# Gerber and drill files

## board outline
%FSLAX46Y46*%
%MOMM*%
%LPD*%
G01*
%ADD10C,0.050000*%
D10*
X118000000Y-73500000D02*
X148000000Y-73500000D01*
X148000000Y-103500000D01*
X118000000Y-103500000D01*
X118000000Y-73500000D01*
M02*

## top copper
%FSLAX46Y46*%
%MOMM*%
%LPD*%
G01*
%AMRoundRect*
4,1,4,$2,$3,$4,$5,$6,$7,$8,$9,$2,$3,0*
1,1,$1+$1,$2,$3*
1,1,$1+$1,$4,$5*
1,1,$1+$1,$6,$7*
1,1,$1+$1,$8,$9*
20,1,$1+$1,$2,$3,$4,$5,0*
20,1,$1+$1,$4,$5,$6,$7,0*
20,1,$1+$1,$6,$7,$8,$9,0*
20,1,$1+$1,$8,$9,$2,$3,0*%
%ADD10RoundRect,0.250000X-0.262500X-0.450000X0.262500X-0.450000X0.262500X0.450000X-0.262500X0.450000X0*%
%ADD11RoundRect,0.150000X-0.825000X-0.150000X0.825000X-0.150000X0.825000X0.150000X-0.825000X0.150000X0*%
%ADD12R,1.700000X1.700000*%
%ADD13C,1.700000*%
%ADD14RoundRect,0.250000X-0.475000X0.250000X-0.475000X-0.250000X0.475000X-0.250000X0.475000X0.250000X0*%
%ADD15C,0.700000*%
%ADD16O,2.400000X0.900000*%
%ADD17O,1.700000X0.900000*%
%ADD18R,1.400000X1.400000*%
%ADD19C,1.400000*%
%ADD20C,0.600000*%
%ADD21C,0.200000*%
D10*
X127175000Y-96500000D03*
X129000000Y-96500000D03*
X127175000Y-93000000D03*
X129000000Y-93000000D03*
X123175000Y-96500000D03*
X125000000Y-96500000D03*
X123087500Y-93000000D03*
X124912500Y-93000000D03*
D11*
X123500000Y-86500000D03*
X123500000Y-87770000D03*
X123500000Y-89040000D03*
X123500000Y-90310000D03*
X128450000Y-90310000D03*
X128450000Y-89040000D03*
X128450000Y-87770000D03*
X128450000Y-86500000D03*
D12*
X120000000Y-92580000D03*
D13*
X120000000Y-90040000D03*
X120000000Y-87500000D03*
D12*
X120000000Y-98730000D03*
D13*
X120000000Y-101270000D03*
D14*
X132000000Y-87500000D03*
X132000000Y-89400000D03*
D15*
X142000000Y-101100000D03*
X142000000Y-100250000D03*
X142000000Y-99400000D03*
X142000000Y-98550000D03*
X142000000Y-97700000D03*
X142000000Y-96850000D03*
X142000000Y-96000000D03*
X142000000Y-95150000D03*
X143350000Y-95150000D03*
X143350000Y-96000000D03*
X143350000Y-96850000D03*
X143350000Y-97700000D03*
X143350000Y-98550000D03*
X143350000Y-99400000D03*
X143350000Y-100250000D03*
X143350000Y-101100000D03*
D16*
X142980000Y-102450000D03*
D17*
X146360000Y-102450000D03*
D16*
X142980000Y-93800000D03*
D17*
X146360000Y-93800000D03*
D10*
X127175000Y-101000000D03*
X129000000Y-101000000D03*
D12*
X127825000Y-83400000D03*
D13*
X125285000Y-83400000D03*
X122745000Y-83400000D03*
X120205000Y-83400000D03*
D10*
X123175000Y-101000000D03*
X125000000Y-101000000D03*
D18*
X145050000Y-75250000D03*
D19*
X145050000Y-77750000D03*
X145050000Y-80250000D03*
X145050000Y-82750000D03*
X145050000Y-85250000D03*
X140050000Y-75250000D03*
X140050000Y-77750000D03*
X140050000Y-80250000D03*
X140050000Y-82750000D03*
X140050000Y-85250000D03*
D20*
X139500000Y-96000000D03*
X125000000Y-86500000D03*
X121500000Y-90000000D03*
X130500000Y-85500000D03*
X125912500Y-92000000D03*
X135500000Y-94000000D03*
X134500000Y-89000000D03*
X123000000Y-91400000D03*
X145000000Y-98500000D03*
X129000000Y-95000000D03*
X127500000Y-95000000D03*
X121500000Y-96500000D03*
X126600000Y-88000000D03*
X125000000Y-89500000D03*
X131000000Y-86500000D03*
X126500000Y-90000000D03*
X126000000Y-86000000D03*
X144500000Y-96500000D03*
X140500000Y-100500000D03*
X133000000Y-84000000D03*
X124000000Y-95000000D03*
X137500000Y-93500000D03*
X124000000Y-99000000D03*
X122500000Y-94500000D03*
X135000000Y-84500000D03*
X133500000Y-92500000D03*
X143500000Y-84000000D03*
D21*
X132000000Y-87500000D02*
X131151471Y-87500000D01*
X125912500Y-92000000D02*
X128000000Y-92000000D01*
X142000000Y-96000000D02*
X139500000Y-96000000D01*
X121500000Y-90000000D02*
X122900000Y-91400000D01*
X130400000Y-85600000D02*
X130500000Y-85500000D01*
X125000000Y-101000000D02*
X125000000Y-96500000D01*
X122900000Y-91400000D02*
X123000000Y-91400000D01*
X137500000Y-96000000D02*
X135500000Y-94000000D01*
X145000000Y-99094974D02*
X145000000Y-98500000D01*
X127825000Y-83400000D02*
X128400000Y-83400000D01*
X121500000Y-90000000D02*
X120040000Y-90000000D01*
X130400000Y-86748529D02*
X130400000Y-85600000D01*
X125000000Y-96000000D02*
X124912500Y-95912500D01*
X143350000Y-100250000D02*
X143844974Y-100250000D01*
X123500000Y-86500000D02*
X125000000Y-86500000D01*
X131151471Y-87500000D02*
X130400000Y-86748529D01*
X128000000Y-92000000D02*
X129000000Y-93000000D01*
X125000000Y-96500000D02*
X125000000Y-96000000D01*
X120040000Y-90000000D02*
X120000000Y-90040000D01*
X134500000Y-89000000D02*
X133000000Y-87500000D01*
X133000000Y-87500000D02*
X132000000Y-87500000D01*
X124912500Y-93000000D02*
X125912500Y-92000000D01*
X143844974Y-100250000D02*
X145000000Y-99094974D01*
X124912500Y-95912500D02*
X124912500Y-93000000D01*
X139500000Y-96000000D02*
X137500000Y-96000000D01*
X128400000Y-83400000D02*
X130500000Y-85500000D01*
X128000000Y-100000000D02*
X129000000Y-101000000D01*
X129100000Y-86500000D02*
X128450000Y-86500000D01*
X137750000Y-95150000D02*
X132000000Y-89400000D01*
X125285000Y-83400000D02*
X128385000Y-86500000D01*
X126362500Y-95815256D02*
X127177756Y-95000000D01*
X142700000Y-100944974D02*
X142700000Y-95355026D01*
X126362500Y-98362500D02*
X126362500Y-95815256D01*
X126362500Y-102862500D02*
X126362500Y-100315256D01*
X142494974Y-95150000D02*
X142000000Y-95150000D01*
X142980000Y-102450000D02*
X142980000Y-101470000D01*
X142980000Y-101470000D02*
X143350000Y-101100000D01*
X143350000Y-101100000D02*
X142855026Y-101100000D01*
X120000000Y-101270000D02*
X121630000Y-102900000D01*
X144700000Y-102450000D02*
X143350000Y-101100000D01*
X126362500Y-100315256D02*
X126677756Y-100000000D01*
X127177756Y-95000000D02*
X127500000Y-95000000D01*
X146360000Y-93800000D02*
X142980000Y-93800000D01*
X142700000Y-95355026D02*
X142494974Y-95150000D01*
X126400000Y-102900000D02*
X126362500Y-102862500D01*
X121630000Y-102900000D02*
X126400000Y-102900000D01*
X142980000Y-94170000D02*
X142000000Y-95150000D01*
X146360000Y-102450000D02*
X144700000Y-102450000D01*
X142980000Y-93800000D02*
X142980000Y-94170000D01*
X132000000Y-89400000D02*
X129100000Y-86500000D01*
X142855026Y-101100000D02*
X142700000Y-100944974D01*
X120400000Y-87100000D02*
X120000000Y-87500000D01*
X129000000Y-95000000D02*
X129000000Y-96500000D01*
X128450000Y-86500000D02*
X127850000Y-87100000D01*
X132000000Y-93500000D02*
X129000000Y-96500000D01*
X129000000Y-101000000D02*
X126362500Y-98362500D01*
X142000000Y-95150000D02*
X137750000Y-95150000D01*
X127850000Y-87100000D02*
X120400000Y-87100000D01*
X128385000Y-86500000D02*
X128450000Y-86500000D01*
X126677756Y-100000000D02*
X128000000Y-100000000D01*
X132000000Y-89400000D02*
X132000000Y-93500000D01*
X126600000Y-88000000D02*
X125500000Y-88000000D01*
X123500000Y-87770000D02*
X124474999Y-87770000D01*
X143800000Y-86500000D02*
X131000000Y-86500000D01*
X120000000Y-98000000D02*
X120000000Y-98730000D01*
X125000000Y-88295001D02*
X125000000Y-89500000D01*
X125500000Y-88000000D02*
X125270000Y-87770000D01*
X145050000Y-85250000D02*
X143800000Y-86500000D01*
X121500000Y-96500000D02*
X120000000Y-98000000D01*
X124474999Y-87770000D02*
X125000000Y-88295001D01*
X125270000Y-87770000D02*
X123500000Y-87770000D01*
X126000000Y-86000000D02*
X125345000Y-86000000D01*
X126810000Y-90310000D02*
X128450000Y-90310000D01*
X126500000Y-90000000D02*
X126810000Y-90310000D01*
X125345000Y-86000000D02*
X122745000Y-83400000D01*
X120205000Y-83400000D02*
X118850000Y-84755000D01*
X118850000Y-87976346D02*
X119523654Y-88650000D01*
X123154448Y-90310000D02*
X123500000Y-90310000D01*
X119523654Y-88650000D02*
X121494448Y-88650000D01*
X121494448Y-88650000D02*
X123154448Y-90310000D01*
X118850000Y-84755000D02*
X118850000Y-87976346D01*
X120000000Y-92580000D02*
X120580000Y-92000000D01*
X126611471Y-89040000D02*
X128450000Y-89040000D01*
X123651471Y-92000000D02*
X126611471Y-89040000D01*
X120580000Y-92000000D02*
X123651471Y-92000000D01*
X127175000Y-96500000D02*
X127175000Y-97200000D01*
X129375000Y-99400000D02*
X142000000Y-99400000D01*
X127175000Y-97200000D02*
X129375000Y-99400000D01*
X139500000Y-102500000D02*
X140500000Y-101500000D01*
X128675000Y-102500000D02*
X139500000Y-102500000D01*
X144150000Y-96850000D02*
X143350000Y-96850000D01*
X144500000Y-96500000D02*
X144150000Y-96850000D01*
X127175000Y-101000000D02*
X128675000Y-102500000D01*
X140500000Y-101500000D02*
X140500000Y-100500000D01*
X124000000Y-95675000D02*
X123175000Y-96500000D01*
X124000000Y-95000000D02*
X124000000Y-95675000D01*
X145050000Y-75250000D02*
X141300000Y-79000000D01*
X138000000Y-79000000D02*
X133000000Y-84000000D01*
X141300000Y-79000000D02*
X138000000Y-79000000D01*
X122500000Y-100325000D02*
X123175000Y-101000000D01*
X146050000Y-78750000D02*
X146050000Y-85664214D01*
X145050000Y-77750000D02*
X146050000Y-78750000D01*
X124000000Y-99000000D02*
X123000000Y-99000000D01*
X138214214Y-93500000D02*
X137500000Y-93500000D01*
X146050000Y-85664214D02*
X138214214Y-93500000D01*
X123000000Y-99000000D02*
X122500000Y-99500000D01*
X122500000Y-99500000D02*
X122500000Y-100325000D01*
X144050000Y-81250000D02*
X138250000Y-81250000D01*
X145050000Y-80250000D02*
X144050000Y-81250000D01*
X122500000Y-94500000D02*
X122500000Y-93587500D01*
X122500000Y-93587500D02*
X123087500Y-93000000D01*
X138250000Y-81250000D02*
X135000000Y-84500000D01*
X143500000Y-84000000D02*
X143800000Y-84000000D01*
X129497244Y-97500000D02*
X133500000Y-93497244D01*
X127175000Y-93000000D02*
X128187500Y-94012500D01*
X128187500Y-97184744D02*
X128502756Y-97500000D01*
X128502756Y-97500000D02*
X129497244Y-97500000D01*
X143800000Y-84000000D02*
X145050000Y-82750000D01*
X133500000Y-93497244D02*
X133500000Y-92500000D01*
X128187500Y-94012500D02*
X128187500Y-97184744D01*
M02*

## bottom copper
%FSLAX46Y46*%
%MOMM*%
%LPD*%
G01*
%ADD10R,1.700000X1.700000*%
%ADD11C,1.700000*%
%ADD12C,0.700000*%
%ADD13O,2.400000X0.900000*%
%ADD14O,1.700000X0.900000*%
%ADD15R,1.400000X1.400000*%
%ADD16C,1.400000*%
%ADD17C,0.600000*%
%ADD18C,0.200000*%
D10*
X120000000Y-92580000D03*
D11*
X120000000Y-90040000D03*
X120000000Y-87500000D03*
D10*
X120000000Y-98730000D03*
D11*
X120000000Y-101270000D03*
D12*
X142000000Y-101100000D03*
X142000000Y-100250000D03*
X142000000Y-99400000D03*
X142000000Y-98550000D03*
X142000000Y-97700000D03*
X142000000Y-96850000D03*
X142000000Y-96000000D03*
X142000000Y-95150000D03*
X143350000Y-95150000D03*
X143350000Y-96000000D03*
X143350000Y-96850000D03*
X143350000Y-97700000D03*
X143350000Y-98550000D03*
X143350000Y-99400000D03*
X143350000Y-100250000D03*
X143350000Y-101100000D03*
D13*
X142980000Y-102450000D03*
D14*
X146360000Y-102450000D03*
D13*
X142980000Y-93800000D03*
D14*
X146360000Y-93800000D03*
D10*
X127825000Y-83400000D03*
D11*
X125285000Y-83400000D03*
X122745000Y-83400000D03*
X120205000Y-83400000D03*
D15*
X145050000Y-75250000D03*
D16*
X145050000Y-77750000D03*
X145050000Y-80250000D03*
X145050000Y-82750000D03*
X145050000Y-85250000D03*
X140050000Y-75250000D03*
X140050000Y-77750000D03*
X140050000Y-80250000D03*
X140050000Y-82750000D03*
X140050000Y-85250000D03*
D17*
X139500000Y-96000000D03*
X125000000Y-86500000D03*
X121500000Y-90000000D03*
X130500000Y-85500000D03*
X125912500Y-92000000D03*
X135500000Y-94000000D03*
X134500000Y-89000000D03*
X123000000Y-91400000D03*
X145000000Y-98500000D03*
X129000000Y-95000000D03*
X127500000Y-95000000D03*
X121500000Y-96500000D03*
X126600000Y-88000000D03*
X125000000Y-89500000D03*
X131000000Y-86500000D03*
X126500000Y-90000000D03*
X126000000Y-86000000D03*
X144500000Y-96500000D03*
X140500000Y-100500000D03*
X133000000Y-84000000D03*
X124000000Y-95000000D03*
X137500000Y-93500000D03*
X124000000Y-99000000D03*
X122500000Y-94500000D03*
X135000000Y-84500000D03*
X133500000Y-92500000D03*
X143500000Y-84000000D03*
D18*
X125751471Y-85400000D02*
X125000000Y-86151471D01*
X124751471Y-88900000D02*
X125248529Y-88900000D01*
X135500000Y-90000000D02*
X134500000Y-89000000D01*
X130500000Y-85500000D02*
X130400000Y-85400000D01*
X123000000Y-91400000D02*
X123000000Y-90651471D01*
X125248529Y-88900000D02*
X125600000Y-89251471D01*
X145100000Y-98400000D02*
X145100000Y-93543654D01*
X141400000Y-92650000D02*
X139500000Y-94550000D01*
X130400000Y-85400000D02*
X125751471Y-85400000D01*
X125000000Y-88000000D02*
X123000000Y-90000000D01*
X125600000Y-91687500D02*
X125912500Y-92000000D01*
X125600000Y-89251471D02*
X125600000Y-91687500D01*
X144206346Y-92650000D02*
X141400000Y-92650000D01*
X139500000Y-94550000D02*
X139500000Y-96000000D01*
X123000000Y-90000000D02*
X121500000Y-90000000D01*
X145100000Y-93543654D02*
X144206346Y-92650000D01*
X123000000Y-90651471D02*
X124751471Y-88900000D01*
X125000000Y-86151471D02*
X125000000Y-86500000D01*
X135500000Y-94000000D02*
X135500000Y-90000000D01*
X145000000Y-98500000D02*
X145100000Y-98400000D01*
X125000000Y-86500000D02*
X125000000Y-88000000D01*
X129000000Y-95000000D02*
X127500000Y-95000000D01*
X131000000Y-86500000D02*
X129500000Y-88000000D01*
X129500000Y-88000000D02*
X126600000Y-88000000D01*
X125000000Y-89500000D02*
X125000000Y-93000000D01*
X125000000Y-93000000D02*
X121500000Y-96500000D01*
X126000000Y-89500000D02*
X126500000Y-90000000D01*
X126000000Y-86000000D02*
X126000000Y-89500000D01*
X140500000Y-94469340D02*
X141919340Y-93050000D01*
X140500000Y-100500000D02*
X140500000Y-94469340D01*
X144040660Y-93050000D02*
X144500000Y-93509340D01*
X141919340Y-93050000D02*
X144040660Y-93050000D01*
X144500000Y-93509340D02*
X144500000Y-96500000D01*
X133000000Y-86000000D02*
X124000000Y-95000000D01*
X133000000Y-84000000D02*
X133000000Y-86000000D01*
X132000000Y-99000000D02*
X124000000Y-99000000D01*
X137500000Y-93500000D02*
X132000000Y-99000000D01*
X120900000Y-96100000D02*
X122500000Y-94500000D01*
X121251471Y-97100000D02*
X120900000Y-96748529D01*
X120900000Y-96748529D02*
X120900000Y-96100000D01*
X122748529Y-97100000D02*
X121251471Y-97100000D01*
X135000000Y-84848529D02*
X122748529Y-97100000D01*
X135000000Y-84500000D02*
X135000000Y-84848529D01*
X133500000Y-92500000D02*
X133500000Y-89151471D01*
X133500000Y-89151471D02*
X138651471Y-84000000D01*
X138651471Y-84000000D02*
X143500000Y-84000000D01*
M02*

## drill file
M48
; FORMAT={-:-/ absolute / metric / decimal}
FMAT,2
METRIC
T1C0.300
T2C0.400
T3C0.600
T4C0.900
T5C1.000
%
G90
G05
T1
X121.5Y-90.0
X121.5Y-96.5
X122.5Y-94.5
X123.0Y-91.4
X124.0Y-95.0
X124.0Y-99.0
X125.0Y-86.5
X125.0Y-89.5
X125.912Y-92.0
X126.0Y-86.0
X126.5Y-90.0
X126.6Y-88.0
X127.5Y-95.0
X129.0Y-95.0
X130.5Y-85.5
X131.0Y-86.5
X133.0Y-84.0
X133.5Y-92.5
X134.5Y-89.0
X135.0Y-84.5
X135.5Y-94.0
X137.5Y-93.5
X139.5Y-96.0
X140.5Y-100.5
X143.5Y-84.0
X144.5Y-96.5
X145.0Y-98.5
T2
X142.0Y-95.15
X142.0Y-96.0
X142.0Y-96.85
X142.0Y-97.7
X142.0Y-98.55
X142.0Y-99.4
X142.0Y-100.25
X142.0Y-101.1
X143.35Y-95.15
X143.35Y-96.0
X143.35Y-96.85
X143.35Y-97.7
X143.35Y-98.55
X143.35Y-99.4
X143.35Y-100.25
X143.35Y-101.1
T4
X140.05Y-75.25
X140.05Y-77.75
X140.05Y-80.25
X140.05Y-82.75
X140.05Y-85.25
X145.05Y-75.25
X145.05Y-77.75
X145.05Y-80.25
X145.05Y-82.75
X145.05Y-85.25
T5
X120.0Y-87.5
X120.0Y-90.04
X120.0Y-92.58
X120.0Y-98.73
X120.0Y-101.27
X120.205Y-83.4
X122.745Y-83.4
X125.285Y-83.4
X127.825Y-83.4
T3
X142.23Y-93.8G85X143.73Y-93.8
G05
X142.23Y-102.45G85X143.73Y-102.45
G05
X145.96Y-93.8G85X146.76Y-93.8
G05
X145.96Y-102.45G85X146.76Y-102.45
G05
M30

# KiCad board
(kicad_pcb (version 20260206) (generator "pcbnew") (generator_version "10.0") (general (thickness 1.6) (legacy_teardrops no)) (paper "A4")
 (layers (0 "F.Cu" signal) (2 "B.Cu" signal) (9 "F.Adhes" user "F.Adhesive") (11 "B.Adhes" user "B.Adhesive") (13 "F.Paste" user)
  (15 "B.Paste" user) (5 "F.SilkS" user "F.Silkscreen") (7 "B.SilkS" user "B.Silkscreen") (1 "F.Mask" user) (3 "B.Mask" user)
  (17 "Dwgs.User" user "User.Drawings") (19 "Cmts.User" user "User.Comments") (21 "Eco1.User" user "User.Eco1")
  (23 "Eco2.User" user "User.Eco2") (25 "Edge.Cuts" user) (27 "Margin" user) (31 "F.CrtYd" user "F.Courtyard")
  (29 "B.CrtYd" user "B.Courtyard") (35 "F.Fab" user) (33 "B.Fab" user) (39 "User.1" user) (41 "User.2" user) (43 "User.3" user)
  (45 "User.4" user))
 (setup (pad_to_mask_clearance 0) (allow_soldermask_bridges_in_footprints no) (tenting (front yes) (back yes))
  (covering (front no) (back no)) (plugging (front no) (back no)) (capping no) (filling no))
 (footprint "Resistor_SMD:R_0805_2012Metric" (layer "F.Cu") (at 128.0875 96.5)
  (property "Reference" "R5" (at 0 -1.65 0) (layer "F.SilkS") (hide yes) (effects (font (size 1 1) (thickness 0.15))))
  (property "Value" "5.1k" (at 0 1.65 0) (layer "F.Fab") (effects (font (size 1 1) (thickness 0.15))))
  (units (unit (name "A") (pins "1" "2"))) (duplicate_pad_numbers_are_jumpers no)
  (pad "1" smd roundrect (at -0.9125 0) (size 1.025 1.4) (layers "F.Cu" "F.Mask" "F.Paste") (roundrect_rratio 0.243902) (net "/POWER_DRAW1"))
  (pad "2" smd roundrect (at 0.9125 0) (size 1.025 1.4) (layers "F.Cu" "F.Mask" "F.Paste") (roundrect_rratio 0.243902) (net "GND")))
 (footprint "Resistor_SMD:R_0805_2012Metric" (layer "F.Cu") (at 128.0875 93)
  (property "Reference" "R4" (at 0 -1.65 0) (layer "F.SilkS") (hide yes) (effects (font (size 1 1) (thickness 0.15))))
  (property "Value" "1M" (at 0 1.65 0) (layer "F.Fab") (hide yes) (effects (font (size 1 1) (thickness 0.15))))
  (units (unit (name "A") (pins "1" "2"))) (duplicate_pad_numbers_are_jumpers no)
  (pad "1" smd roundrect (at -0.9125 0) (size 1.025 1.4) (layers "F.Cu" "F.Mask" "F.Paste") (roundrect_rratio 0.243902)
   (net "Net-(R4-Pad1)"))
  (pad "2" smd roundrect (at 0.9125 0) (size 1.025 1.4) (layers "F.Cu" "F.Mask" "F.Paste") (roundrect_rratio 0.243902) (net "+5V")))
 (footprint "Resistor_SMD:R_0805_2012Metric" (layer "F.Cu") (at 124.0875 96.5)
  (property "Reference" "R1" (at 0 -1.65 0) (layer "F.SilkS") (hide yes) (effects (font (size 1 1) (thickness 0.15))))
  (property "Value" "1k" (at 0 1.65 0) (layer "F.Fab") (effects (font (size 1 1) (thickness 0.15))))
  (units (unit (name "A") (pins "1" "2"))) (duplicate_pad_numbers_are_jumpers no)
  (pad "1" smd roundrect (at -0.9125 0) (size 1.025 1.4) (layers "F.Cu" "F.Mask" "F.Paste") (roundrect_rratio 0.243902)
   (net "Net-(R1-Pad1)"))
  (pad "2" smd roundrect (at 0.9125 0) (size 1.025 1.4) (layers "F.Cu" "F.Mask" "F.Paste") (roundrect_rratio 0.243902) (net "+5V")))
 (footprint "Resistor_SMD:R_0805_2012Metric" (layer "F.Cu") (at 124 93)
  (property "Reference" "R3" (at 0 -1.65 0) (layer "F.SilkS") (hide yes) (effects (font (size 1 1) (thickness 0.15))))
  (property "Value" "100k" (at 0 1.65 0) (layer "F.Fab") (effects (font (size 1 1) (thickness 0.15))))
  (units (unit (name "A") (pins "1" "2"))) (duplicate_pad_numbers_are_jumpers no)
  (pad "1" smd roundrect (at -0.9125 0) (size 1.025 1.4) (layers "F.Cu" "F.Mask" "F.Paste") (roundrect_rratio 0.243902)
   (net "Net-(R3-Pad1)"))
  (pad "2" smd roundrect (at 0.9125 0) (size 1.025 1.4) (layers "F.Cu" "F.Mask" "F.Paste") (roundrect_rratio 0.243902) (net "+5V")))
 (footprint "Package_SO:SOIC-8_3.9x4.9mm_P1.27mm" (layer "F.Cu") (at 125.975 88.405)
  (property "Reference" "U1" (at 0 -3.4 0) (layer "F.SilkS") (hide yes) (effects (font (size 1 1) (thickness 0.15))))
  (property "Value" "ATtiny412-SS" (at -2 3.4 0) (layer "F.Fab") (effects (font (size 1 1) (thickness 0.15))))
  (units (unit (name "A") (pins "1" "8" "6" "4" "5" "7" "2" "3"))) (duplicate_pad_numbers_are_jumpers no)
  (pad "1" smd roundrect (at -2.475 -1.905) (size 1.95 0.6) (layers "F.Cu" "F.Mask" "F.Paste") (roundrect_rratio 0.25) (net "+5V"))
  (pad "2" smd roundrect (at -2.475 -0.635) (size 1.95 0.6) (layers "F.Cu" "F.Mask" "F.Paste") (roundrect_rratio 0.25) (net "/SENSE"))
  (pad "3" smd roundrect (at -2.475 0.635) (size 1.95 0.6) (layers "F.Cu" "F.Mask" "F.Paste") (roundrect_rratio 0.25)
   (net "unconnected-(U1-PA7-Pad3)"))
  (pad "4" smd roundrect (at -2.475 1.905) (size 1.95 0.6) (layers "F.Cu" "F.Mask" "F.Paste") (roundrect_rratio 0.25) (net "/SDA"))
  (pad "5" smd roundrect (at 2.475 1.905) (size 1.95 0.6) (layers "F.Cu" "F.Mask" "F.Paste") (roundrect_rratio 0.25) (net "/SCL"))
  (pad "6" smd roundrect (at 2.475 0.635) (size 1.95 0.6) (layers "F.Cu" "F.Mask" "F.Paste") (roundrect_rratio 0.25) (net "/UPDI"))
  (pad "7" smd roundrect (at 2.475 -0.635) (size 1.95 0.6) (layers "F.Cu" "F.Mask" "F.Paste") (roundrect_rratio 0.25)
   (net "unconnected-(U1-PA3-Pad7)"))
  (pad "8" smd roundrect (at 2.475 -1.905) (size 1.95 0.6) (layers "F.Cu" "F.Mask" "F.Paste") (roundrect_rratio 0.25) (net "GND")))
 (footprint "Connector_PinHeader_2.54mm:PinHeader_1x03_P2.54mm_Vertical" (layer "F.Cu") (at 120 92.58 180)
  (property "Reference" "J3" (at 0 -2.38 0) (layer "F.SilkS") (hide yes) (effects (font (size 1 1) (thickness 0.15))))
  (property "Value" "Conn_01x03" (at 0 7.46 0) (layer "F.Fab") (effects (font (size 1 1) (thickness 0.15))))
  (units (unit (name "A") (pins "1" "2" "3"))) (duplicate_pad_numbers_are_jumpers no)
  (pad "1" thru_hole rect (at 0 0 180) (size 1.7 1.7) (drill 1) (layers "*.Cu" "*.Mask") (remove_unused_layers no) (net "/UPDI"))
  (pad "2" thru_hole circle (at 0 2.54 180) (size 1.7 1.7) (drill 1) (layers "*.Cu" "*.Mask") (remove_unused_layers no) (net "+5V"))
  (pad "3" thru_hole circle (at 0 5.08 180) (size 1.7 1.7) (drill 1) (layers "*.Cu" "*.Mask") (remove_unused_layers no) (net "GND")))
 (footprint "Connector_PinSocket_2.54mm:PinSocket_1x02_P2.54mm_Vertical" (layer "F.Cu") (at 120 98.73)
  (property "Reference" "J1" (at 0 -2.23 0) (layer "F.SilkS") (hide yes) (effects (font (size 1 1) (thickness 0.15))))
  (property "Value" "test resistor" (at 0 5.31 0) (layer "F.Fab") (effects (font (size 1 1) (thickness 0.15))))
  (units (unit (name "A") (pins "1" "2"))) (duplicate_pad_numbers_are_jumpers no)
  (pad "1" thru_hole rect (at 0 0) (size 1.7 1.7) (drill 1) (layers "*.Cu" "*.Mask") (remove_unused_layers no) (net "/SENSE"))
  (pad "2" thru_hole circle (at 0 2.54) (size 1.7 1.7) (drill 1) (layers "*.Cu" "*.Mask") (remove_unused_layers no) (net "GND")))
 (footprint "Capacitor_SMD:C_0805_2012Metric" (layer "F.Cu") (at 132 88.45 -90)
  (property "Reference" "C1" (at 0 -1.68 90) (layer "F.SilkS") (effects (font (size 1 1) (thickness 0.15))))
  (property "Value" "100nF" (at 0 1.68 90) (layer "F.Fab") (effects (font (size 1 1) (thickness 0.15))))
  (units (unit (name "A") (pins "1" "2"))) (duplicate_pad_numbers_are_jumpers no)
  (pad "1" smd roundrect (at -0.95 0 270) (size 1 1.45) (layers "F.Cu" "F.Mask" "F.Paste") (roundrect_rratio 0.25) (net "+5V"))
  (pad "2" smd roundrect (at 0.95 0 270) (size 1 1.45) (layers "F.Cu" "F.Mask" "F.Paste") (roundrect_rratio 0.25) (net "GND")))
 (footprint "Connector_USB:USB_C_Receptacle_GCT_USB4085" (layer "F.Cu") (at 142 101.1 90)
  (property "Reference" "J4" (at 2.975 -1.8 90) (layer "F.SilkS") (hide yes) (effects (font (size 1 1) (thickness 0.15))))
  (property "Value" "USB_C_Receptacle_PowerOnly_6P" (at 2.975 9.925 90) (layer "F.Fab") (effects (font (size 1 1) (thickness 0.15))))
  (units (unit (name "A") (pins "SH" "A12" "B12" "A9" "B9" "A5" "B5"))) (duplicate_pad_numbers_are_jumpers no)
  (pad "A1" thru_hole circle (at 0 0 90) (size 0.7 0.7) (drill 0.4) (layers "*.Cu" "*.Mask") (remove_unused_layers no))
  (pad "A4" thru_hole circle (at 0.85 0 90) (size 0.7 0.7) (drill 0.4) (layers "*.Cu" "*.Mask") (remove_unused_layers no))
  (pad "A5" thru_hole circle (at 1.7 0 90) (size 0.7 0.7) (drill 0.4) (layers "*.Cu" "*.Mask") (remove_unused_layers no)
   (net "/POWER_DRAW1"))
  (pad "A6" thru_hole circle (at 2.55 0 90) (size 0.7 0.7) (drill 0.4) (layers "*.Cu" "*.Mask") (remove_unused_layers no))
  (pad "A7" thru_hole circle (at 3.4 0 90) (size 0.7 0.7) (drill 0.4) (layers "*.Cu" "*.Mask") (remove_unused_layers no))
  (pad "A8" thru_hole circle (at 4.25 0 90) (size 0.7 0.7) (drill 0.4) (layers "*.Cu" "*.Mask") (remove_unused_layers no))
  (pad "A9" thru_hole circle (at 5.1 0 90) (size 0.7 0.7) (drill 0.4) (layers "*.Cu" "*.Mask") (remove_unused_layers no) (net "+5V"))
  (pad "A12" thru_hole circle (at 5.95 0 90) (size 0.7 0.7) (drill 0.4) (layers "*.Cu" "*.Mask") (remove_unused_layers no) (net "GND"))
  (pad "B1" thru_hole circle (at 5.95 1.35 90) (size 0.7 0.7) (drill 0.4) (layers "*.Cu" "*.Mask") (remove_unused_layers no))
  (pad "B4" thru_hole circle (at 5.1 1.35 90) (size 0.7 0.7) (drill 0.4) (layers "*.Cu" "*.Mask") (remove_unused_layers no))
  (pad "B5" thru_hole circle (at 4.25 1.35 90) (size 0.7 0.7) (drill 0.4) (layers "*.Cu" "*.Mask") (remove_unused_layers no)
   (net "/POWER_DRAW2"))
  (pad "B6" thru_hole circle (at 3.4 1.35 90) (size 0.7 0.7) (drill 0.4) (layers "*.Cu" "*.Mask") (remove_unused_layers no))
  (pad "B7" thru_hole circle (at 2.55 1.35 90) (size 0.7 0.7) (drill 0.4) (layers "*.Cu" "*.Mask") (remove_unused_layers no))
  (pad "B8" thru_hole circle (at 1.7 1.35 90) (size 0.7 0.7) (drill 0.4) (layers "*.Cu" "*.Mask") (remove_unused_layers no))
  (pad "B9" thru_hole circle (at 0.85 1.35 90) (size 0.7 0.7) (drill 0.4) (layers "*.Cu" "*.Mask") (remove_unused_layers no) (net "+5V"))
  (pad "B12" thru_hole circle (at 0 1.35 90) (size 0.7 0.7) (drill 0.4) (layers "*.Cu" "*.Mask") (remove_unused_layers no) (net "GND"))
  (pad "SH" thru_hole oval (at -1.35 0.98 90) (size 0.9 2.4) (drill oval 0.6 2.1) (layers "*.Cu" "*.Mask") (remove_unused_layers no)
   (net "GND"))
  (pad "SH" thru_hole oval (at -1.35 4.36 90) (size 0.9 1.7) (drill oval 0.6 1.4) (layers "*.Cu" "*.Mask") (remove_unused_layers no)
   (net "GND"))
  (pad "SH" thru_hole oval (at 7.3 0.98 90) (size 0.9 2.4) (drill oval 0.6 2.1) (layers "*.Cu" "*.Mask") (remove_unused_layers no)
   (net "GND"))
  (pad "SH" thru_hole oval (at 7.3 4.36 90) (size 0.9 1.7) (drill oval 0.6 1.4) (layers "*.Cu" "*.Mask") (remove_unused_layers no)
   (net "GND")))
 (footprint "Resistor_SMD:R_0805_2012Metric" (layer "F.Cu") (at 128.0875 101)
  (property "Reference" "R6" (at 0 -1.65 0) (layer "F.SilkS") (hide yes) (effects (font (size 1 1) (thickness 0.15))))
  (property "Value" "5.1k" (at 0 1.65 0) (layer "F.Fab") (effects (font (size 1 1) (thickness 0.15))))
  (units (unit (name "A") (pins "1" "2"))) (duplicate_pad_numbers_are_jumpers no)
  (pad "1" smd roundrect (at -0.9125 0) (size 1.025 1.4) (layers "F.Cu" "F.Mask" "F.Paste") (roundrect_rratio 0.243902) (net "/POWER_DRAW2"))
  (pad "2" smd roundrect (at 0.9125 0) (size 1.025 1.4) (layers "F.Cu" "F.Mask" "F.Paste") (roundrect_rratio 0.243902) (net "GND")))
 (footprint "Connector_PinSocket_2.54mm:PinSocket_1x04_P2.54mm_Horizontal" (layer "F.Cu") (at 127.825 83.4 -90)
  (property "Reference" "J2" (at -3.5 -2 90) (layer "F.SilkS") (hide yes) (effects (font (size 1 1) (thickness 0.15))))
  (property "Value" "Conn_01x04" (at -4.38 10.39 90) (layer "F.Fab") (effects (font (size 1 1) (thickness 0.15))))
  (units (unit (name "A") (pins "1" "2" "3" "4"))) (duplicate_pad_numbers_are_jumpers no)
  (pad "1" thru_hole rect (at 0 0 270) (size 1.7 1.7) (drill 1) (layers "*.Cu" "*.Mask") (remove_unused_layers no) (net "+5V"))
  (pad "2" thru_hole circle (at 0 2.54 270) (size 1.7 1.7) (drill 1) (layers "*.Cu" "*.Mask") (remove_unused_layers no) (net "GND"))
  (pad "3" thru_hole circle (at 0 5.08 270) (size 1.7 1.7) (drill 1) (layers "*.Cu" "*.Mask") (remove_unused_layers no) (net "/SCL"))
  (pad "4" thru_hole circle (at 0 7.62 270) (size 1.7 1.7) (drill 1) (layers "*.Cu" "*.Mask") (remove_unused_layers no) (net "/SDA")))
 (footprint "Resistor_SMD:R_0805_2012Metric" (layer "F.Cu") (at 124.0875 101)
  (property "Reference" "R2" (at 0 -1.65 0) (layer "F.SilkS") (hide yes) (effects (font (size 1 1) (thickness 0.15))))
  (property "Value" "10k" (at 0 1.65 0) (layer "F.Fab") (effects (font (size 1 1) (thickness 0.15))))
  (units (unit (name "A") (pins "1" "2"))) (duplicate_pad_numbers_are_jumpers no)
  (pad "1" smd roundrect (at -0.9125 0) (size 1.025 1.4) (layers "F.Cu" "F.Mask" "F.Paste") (roundrect_rratio 0.243902)
   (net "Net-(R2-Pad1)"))
  (pad "2" smd roundrect (at 0.9125 0) (size 1.025 1.4) (layers "F.Cu" "F.Mask" "F.Paste") (roundrect_rratio 0.243902) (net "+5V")))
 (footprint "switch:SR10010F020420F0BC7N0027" (layer "F.Cu") (at 145.05 75.25)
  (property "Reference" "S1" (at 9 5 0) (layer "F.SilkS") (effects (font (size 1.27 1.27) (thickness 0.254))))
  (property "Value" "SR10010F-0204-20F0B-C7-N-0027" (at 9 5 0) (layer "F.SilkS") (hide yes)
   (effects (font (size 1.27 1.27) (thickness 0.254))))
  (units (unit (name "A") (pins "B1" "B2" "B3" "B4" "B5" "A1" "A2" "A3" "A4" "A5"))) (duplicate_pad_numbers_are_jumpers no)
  (pad "A1" thru_hole rect (at 0 0) (size 1.4 1.4) (drill 0.9) (layers "*.Cu" "*.Mask") (remove_unused_layers no) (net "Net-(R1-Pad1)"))
  (pad "A2" thru_hole circle (at 0 2.5) (size 1.4 1.4) (drill 0.9) (layers "*.Cu" "*.Mask") (remove_unused_layers no) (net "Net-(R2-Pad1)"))
  (pad "A3" thru_hole circle (at 0 5) (size 1.4 1.4) (drill 0.9) (layers "*.Cu" "*.Mask") (remove_unused_layers no) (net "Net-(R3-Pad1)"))
  (pad "A4" thru_hole circle (at 0 7.5) (size 1.4 1.4) (drill 0.9) (layers "*.Cu" "*.Mask") (remove_unused_layers no) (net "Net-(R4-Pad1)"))
  (pad "A5" thru_hole circle (at 0 10) (size 1.4 1.4) (drill 0.9) (layers "*.Cu" "*.Mask") (remove_unused_layers no) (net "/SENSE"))
  (pad "B1" thru_hole circle (at -5 0) (size 1.4 1.4) (drill 0.9) (layers "*.Cu" "*.Mask") (remove_unused_layers no)
   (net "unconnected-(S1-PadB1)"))
  (pad "B2" thru_hole circle (at -5 2.5) (size 1.4 1.4) (drill 0.9) (layers "*.Cu" "*.Mask") (remove_unused_layers no)
   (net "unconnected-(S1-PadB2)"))
  (pad "B3" thru_hole circle (at -5 5) (size 1.4 1.4) (drill 0.9) (layers "*.Cu" "*.Mask") (remove_unused_layers no)
   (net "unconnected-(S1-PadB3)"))
  (pad "B4" thru_hole circle (at -5 7.5) (size 1.4 1.4) (drill 0.9) (layers "*.Cu" "*.Mask") (remove_unused_layers no)
   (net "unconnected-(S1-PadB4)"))
  (pad "B5" thru_hole circle (at -5 10) (size 1.4 1.4) (drill 0.9) (layers "*.Cu" "*.Mask") (remove_unused_layers no)
   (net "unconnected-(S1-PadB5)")))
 (gr_rect (start 118 73.5) (end 148 103.5) (stroke (width 0.05) (type default)) (fill no) (layer "Edge.Cuts"))
 (segment (start 132 87.5) (end 131.151471 87.5) (width 0.2) (layer "F.Cu") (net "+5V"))
 (segment (start 125.9125 92) (end 128 92) (width 0.2) (layer "F.Cu") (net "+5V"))
 (segment (start 142 96) (end 139.5 96) (width 0.2) (layer "F.Cu") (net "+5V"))
 (segment (start 121.5 90) (end 122.9 91.4) (width 0.2) (layer "F.Cu") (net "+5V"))
 (segment (start 130.4 85.6) (end 130.5 85.5) (width 0.2) (layer "F.Cu") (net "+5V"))
 (segment (start 125 101) (end 125 96.5) (width 0.2) (layer "F.Cu") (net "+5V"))
 (segment (start 122.9 91.4) (end 123 91.4) (width 0.2) (layer "F.Cu") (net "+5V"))
 (segment (start 137.5 96) (end 135.5 94) (width 0.2) (layer "F.Cu") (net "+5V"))
 (segment (start 145 99.094974) (end 145 98.5) (width 0.2) (layer "F.Cu") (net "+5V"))
 (segment (start 127.825 83.4) (end 128.4 83.4) (width 0.2) (layer "F.Cu") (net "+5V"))
 (segment (start 121.5 90) (end 120.04 90) (width 0.2) (layer "F.Cu") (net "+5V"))
 (segment (start 130.4 86.748529) (end 130.4 85.6) (width 0.2) (layer "F.Cu") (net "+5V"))
 (segment (start 125 96) (end 124.9125 95.9125) (width 0.2) (layer "F.Cu") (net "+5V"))
 (segment (start 143.35 100.25) (end 143.844974 100.25) (width 0.2) (layer "F.Cu") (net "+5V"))
 (segment (start 123.5 86.5) (end 125 86.5) (width 0.2) (layer "F.Cu") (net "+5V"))
 (segment (start 131.151471 87.5) (end 130.4 86.748529) (width 0.2) (layer "F.Cu") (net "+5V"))
 (segment (start 128 92) (end 129 93) (width 0.2) (layer "F.Cu") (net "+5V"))
 (segment (start 125 96.5) (end 125 96) (width 0.2) (layer "F.Cu") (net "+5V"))
 (segment (start 120.04 90) (end 120 90.04) (width 0.2) (layer "F.Cu") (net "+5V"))
 (segment (start 134.5 89) (end 133 87.5) (width 0.2) (layer "F.Cu") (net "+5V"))
 (segment (start 133 87.5) (end 132 87.5) (width 0.2) (layer "F.Cu") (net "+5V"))
 (segment (start 124.9125 93) (end 125.9125 92) (width 0.2) (layer "F.Cu") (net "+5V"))
 (segment (start 143.844974 100.25) (end 145 99.094974) (width 0.2) (layer "F.Cu") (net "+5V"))
 (segment (start 124.9125 95.9125) (end 124.9125 93) (width 0.2) (layer "F.Cu") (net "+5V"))
 (segment (start 139.5 96) (end 137.5 96) (width 0.2) (layer "F.Cu") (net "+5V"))
 (segment (start 128.4 83.4) (end 130.5 85.5) (width 0.2) (layer "F.Cu") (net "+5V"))
 (via (at 139.5 96) (size 0.6) (drill 0.3) (layers "F.Cu" "B.Cu") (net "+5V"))
 (via (at 125 86.5) (size 0.6) (drill 0.3) (layers "F.Cu" "B.Cu") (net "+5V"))
 (via (at 121.5 90) (size 0.6) (drill 0.3) (layers "F.Cu" "B.Cu") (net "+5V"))
 (via (at 130.5 85.5) (size 0.6) (drill 0.3) (layers "F.Cu" "B.Cu") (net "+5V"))
 (via (at 125.9125 92) (size 0.6) (drill 0.3) (layers "F.Cu" "B.Cu") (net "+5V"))
 (via (at 135.5 94) (size 0.6) (drill 0.3) (layers "F.Cu" "B.Cu") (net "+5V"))
 (via (at 134.5 89) (size 0.6) (drill 0.3) (layers "F.Cu" "B.Cu") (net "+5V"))
 (via (at 123 91.4) (size 0.6) (drill 0.3) (layers "F.Cu" "B.Cu") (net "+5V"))
 (via (at 145 98.5) (size 0.6) (drill 0.3) (layers "F.Cu" "B.Cu") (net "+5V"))
 (segment (start 125.751471 85.4) (end 125 86.151471) (width 0.2) (layer "B.Cu") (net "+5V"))
 (segment (start 124.751471 88.9) (end 125.248529 88.9) (width 0.2) (layer "B.Cu") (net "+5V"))
 (segment (start 135.5 90) (end 134.5 89) (width 0.2) (layer "B.Cu") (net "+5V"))
 (segment (start 130.5 85.5) (end 130.4 85.4) (width 0.2) (layer "B.Cu") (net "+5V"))
 (segment (start 123 91.4) (end 123 90.651471) (width 0.2) (layer "B.Cu") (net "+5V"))
 (segment (start 125.248529 88.9) (end 125.6 89.251471) (width 0.2) (layer "B.Cu") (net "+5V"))
 (segment (start 145.1 98.4) (end 145.1 93.543654) (width 0.2) (layer "B.Cu") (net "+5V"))
 (segment (start 141.4 92.65) (end 139.5 94.55) (width 0.2) (layer "B.Cu") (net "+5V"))
 (segment (start 130.4 85.4) (end 125.751471 85.4) (width 0.2) (layer "B.Cu") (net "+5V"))
 (segment (start 125 88) (end 123 90) (width 0.2) (layer "B.Cu") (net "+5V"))
 (segment (start 125.6 91.6875) (end 125.9125 92) (width 0.2) (layer "B.Cu") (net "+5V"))
 (segment (start 125.6 89.251471) (end 125.6 91.6875) (width 0.2) (layer "B.Cu") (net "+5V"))
 (segment (start 144.206346 92.65) (end 141.4 92.65) (width 0.2) (layer "B.Cu") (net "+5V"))
 (segment (start 139.5 94.55) (end 139.5 96) (width 0.2) (layer "B.Cu") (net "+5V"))
 (segment (start 123 90) (end 121.5 90) (width 0.2) (layer "B.Cu") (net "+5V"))
 (segment (start 145.1 93.543654) (end 144.206346 92.65) (width 0.2) (layer "B.Cu") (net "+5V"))
 (segment (start 123 90.651471) (end 124.751471 88.9) (width 0.2) (layer "B.Cu") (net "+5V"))
 (segment (start 125 86.151471) (end 125 86.5) (width 0.2) (layer "B.Cu") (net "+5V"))
 (segment (start 135.5 94) (end 135.5 90) (width 0.2) (layer "B.Cu") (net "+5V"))
 (segment (start 145 98.5) (end 145.1 98.4) (width 0.2) (layer "B.Cu") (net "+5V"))
 (segment (start 125 86.5) (end 125 88) (width 0.2) (layer "B.Cu") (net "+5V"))
 (segment (start 128 100) (end 129 101) (width 0.2) (layer "F.Cu") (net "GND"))
 (segment (start 129.1 86.5) (end 128.45 86.5) (width 0.2) (layer "F.Cu") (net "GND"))
 (segment (start 137.75 95.15) (end 132 89.4) (width 0.2) (layer "F.Cu") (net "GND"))
 (segment (start 125.285 83.4) (end 128.385 86.5) (width 0.2) (layer "F.Cu") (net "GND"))
 (segment (start 126.3625 95.815256) (end 127.177756 95) (width 0.2) (layer "F.Cu") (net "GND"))
 (segment (start 142.7 100.944974) (end 142.7 95.355026) (width 0.2) (layer "F.Cu") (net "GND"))
 (segment (start 126.3625 98.3625) (end 126.3625 95.815256) (width 0.2) (layer "F.Cu") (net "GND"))
 (segment (start 126.3625 102.8625) (end 126.3625 100.315256) (width 0.2) (layer "F.Cu") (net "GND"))
 (segment (start 142.494974 95.15) (end 142 95.15) (width 0.2) (layer "F.Cu") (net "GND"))
 (segment (start 142.98 102.45) (end 142.98 101.47) (width 0.2) (layer "F.Cu") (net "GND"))
 (segment (start 142.98 101.47) (end 143.35 101.1) (width 0.2) (layer "F.Cu") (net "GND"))
 (segment (start 143.35 101.1) (end 142.855026 101.1) (width 0.2) (layer "F.Cu") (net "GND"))
 (segment (start 120 101.27) (end 121.63 102.9) (width 0.2) (layer "F.Cu") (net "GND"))
 (segment (start 144.7 102.45) (end 143.35 101.1) (width 0.2) (layer "F.Cu") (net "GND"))
 (segment (start 126.3625 100.315256) (end 126.677756 100) (width 0.2) (layer "F.Cu") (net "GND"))
 (segment (start 127.177756 95) (end 127.5 95) (width 0.2) (layer "F.Cu") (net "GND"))
 (segment (start 146.36 93.8) (end 142.98 93.8) (width 0.2) (layer "F.Cu") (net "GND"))
 (segment (start 142.7 95.355026) (end 142.494974 95.15) (width 0.2) (layer "F.Cu") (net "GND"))
 (segment (start 126.4 102.9) (end 126.3625 102.8625) (width 0.2) (layer "F.Cu") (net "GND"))
 (segment (start 121.63 102.9) (end 126.4 102.9) (width 0.2) (layer "F.Cu") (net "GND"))
 (segment (start 142.98 94.17) (end 142 95.15) (width 0.2) (layer "F.Cu") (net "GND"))
 (segment (start 146.36 102.45) (end 144.7 102.45) (width 0.2) (layer "F.Cu") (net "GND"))
 (segment (start 142.98 93.8) (end 142.98 94.17) (width 0.2) (layer "F.Cu") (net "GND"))
 (segment (start 132 89.4) (end 129.1 86.5) (width 0.2) (layer "F.Cu") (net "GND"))
 (segment (start 142.855026 101.1) (end 142.7 100.944974) (width 0.2) (layer "F.Cu") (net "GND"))
 (segment (start 120.4 87.1) (end 120 87.5) (width 0.2) (layer "F.Cu") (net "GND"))
 (segment (start 129 95) (end 129 96.5) (width 0.2) (layer "F.Cu") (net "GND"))
 (segment (start 128.45 86.5) (end 127.85 87.1) (width 0.2) (layer "F.Cu") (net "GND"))
 (segment (start 132 93.5) (end 129 96.5) (width 0.2) (layer "F.Cu") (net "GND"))
 (segment (start 129 101) (end 126.3625 98.3625) (width 0.2) (layer "F.Cu") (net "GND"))
 (segment (start 142 95.15) (end 137.75 95.15) (width 0.2) (layer "F.Cu") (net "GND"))
 (segment (start 127.85 87.1) (end 120.4 87.1) (width 0.2) (layer "F.Cu") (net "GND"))
 (segment (start 128.385 86.5) (end 128.45 86.5) (width 0.2) (layer "F.Cu") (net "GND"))
 (segment (start 126.677756 100) (end 128 100) (width 0.2) (layer "F.Cu") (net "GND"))
 (segment (start 132 89.4) (end 132 93.5) (width 0.2) (layer "F.Cu") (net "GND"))
 (via (at 129 95) (size 0.6) (drill 0.3) (layers "F.Cu" "B.Cu") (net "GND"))
 (via (at 127.5 95) (size 0.6) (drill 0.3) (layers "F.Cu" "B.Cu") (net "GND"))
 (segment (start 129 95) (end 127.5 95) (width 0.2) (layer "B.Cu") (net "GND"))
 (segment (start 126.6 88) (end 125.5 88) (width 0.2) (layer "F.Cu") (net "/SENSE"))
 (segment (start 123.5 87.77) (end 124.474999 87.77) (width 0.2) (layer "F.Cu") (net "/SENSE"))
 (segment (start 143.8 86.5) (end 131 86.5) (width 0.2) (layer "F.Cu") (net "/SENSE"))
 (segment (start 120 98) (end 120 98.73) (width 0.2) (layer "F.Cu") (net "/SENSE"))
 (segment (start 125 88.295001) (end 125 89.5) (width 0.2) (layer "F.Cu") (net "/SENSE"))
 (segment (start 125.5 88) (end 125.27 87.77) (width 0.2) (layer "F.Cu") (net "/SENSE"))
 (segment (start 145.05 85.25) (end 143.8 86.5) (width 0.2) (layer "F.Cu") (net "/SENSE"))
 (segment (start 121.5 96.5) (end 120 98) (width 0.2) (layer "F.Cu") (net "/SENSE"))
 (segment (start 124.474999 87.77) (end 125 88.295001) (width 0.2) (layer "F.Cu") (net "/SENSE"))
 (segment (start 125.27 87.77) (end 123.5 87.77) (width 0.2) (layer "F.Cu") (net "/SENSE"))
 (via (at 121.5 96.5) (size 0.6) (drill 0.3) (layers "F.Cu" "B.Cu") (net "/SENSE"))
 (via (at 126.6 88) (size 0.6) (drill 0.3) (layers "F.Cu" "B.Cu") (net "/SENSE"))
 (via (at 125 89.5) (size 0.6) (drill 0.3) (layers "F.Cu" "B.Cu") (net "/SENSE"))
 (via (at 131 86.5) (size 0.6) (drill 0.3) (layers "F.Cu" "B.Cu") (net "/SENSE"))
 (segment (start 131 86.5) (end 129.5 88) (width 0.2) (layer "B.Cu") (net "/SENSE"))
 (segment (start 129.5 88) (end 126.6 88) (width 0.2) (layer "B.Cu") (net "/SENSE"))
 (segment (start 125 89.5) (end 125 93) (width 0.2) (layer "B.Cu") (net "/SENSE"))
 (segment (start 125 93) (end 121.5 96.5) (width 0.2) (layer "B.Cu") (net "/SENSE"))
 (segment (start 126 86) (end 125.345 86) (width 0.2) (layer "F.Cu") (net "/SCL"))
 (segment (start 126.81 90.31) (end 128.45 90.31) (width 0.2) (layer "F.Cu") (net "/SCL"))
 (segment (start 126.5 90) (end 126.81 90.31) (width 0.2) (layer "F.Cu") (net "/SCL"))
 (segment (start 125.345 86) (end 122.745 83.4) (width 0.2) (layer "F.Cu") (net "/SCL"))
 (via (at 126.5 90) (size 0.6) (drill 0.3) (layers "F.Cu" "B.Cu") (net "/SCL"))
 (via (at 126 86) (size 0.6) (drill 0.3) (layers "F.Cu" "B.Cu") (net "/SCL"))
 (segment (start 126 89.5) (end 126.5 90) (width 0.2) (layer "B.Cu") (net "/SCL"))
 (segment (start 126 86) (end 126 89.5) (width 0.2) (layer "B.Cu") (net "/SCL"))
 (segment (start 120.205 83.4) (end 118.85 84.755) (width 0.2) (layer "F.Cu") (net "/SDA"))
 (segment (start 118.85 87.976346) (end 119.523654 88.65) (width 0.2) (layer "F.Cu") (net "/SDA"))
 (segment (start 123.154448 90.31) (end 123.5 90.31) (width 0.2) (layer "F.Cu") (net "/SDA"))
 (segment (start 119.523654 88.65) (end 121.494448 88.65) (width 0.2) (layer "F.Cu") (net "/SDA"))
 (segment (start 121.494448 88.65) (end 123.154448 90.31) (width 0.2) (layer "F.Cu") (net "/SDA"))
 (segment (start 118.85 84.755) (end 118.85 87.976346) (width 0.2) (layer "F.Cu") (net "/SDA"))
 (segment (start 120 92.58) (end 120.58 92) (width 0.2) (layer "F.Cu") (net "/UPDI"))
 (segment (start 126.611471 89.04) (end 128.45 89.04) (width 0.2) (layer "F.Cu") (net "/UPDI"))
 (segment (start 123.651471 92) (end 126.611471 89.04) (width 0.2) (layer "F.Cu") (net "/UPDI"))
 (segment (start 120.58 92) (end 123.651471 92) (width 0.2) (layer "F.Cu") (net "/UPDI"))
 (segment (start 127.175 96.5) (end 127.175 97.2) (width 0.2) (layer "F.Cu") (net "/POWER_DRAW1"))
 (segment (start 129.375 99.4) (end 142 99.4) (width 0.2) (layer "F.Cu") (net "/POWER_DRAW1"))
 (segment (start 127.175 97.2) (end 129.375 99.4) (width 0.2) (layer "F.Cu") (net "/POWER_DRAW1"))
 (segment (start 139.5 102.5) (end 140.5 101.5) (width 0.2) (layer "F.Cu") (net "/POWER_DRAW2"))
 (segment (start 128.675 102.5) (end 139.5 102.5) (width 0.2) (layer "F.Cu") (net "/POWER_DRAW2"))
 (segment (start 144.15 96.85) (end 143.35 96.85) (width 0.2) (layer "F.Cu") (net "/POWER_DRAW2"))
 (segment (start 144.5 96.5) (end 144.15 96.85) (width 0.2) (layer "F.Cu") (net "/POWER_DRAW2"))
 (segment (start 127.175 101) (end 128.675 102.5) (width 0.2) (layer "F.Cu") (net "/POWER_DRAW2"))
 (segment (start 140.5 101.5) (end 140.5 100.5) (width 0.2) (layer "F.Cu") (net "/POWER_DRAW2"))
 (via (at 144.5 96.5) (size 0.6) (drill 0.3) (layers "F.Cu" "B.Cu") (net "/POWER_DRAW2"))
 (via (at 140.5 100.5) (size 0.6) (drill 0.3) (layers "F.Cu" "B.Cu") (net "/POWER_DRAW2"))
 (segment (start 140.5 94.46934) (end 141.91934 93.05) (width 0.2) (layer "B.Cu") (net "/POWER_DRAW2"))
 (segment (start 140.5 100.5) (end 140.5 94.46934) (width 0.2) (layer "B.Cu") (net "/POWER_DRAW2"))
 (segment (start 144.04066 93.05) (end 144.5 93.50934) (width 0.2) (layer "B.Cu") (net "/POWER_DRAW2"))
 (segment (start 141.91934 93.05) (end 144.04066 93.05) (width 0.2) (layer "B.Cu") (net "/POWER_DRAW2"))
 (segment (start 144.5 93.50934) (end 144.5 96.5) (width 0.2) (layer "B.Cu") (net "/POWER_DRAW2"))
 (segment (start 124 95.675) (end 123.175 96.5) (width 0.2) (layer "F.Cu") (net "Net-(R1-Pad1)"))
 (segment (start 124 95) (end 124 95.675) (width 0.2) (layer "F.Cu") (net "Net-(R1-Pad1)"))
 (segment (start 145.05 75.25) (end 141.3 79) (width 0.2) (layer "F.Cu") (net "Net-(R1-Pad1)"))
 (segment (start 138 79) (end 133 84) (width 0.2) (layer "F.Cu") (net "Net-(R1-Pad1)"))
 (segment (start 141.3 79) (end 138 79) (width 0.2) (layer "F.Cu") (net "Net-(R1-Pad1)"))
 (via (at 133 84) (size 0.6) (drill 0.3) (layers "F.Cu" "B.Cu") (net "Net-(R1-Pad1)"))
 (via (at 124 95) (size 0.6) (drill 0.3) (layers "F.Cu" "B.Cu") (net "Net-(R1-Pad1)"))
 (segment (start 133 86) (end 124 95) (width 0.2) (layer "B.Cu") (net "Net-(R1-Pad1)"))
 (segment (start 133 84) (end 133 86) (width 0.2) (layer "B.Cu") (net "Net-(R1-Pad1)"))
 (segment (start 122.5 100.325) (end 123.175 101) (width 0.2) (layer "F.Cu") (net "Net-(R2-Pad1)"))
 (segment (start 146.05 78.75) (end 146.05 85.664214) (width 0.2) (layer "F.Cu") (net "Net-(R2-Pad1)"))
 (segment (start 145.05 77.75) (end 146.05 78.75) (width 0.2) (layer "F.Cu") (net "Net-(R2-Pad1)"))
 (segment (start 124 99) (end 123 99) (width 0.2) (layer "F.Cu") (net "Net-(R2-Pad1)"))
 (segment (start 138.214214 93.5) (end 137.5 93.5) (width 0.2) (layer "F.Cu") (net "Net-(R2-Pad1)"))
 (segment (start 146.05 85.664214) (end 138.214214 93.5) (width 0.2) (layer "F.Cu") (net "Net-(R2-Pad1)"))
 (segment (start 123 99) (end 122.5 99.5) (width 0.2) (layer "F.Cu") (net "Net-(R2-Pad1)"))
 (segment (start 122.5 99.5) (end 122.5 100.325) (width 0.2) (layer "F.Cu") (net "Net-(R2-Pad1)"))
 (via (at 137.5 93.5) (size 0.6) (drill 0.3) (layers "F.Cu" "B.Cu") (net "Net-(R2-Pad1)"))
 (via (at 124 99) (size 0.6) (drill 0.3) (layers "F.Cu" "B.Cu") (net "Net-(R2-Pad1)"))
 (segment (start 132 99) (end 124 99) (width 0.2) (layer "B.Cu") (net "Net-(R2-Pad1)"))
 (segment (start 137.5 93.5) (end 132 99) (width 0.2) (layer "B.Cu") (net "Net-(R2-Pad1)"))
 (segment (start 144.05 81.25) (end 138.25 81.25) (width 0.2) (layer "F.Cu") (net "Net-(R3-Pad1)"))
 (segment (start 145.05 80.25) (end 144.05 81.25) (width 0.2) (layer "F.Cu") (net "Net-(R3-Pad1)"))
 (segment (start 122.5 94.5) (end 122.5 93.5875) (width 0.2) (layer "F.Cu") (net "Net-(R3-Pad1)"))
 (segment (start 122.5 93.5875) (end 123.0875 93) (width 0.2) (layer "F.Cu") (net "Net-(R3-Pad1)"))
 (segment (start 138.25 81.25) (end 135 84.5) (width 0.2) (layer "F.Cu") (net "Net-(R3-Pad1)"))
 (via (at 122.5 94.5) (size 0.6) (drill 0.3) (layers "F.Cu" "B.Cu") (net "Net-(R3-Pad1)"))
 (via (at 135 84.5) (size 0.6) (drill 0.3) (layers "F.Cu" "B.Cu") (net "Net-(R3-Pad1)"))
 (segment (start 120.9 96.1) (end 122.5 94.5) (width 0.2) (layer "B.Cu") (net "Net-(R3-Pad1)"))
 (segment (start 121.251471 97.1) (end 120.9 96.748529) (width 0.2) (layer "B.Cu") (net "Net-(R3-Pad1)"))
 (segment (start 120.9 96.748529) (end 120.9 96.1) (width 0.2) (layer "B.Cu") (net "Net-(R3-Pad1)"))
 (segment (start 122.748529 97.1) (end 121.251471 97.1) (width 0.2) (layer "B.Cu") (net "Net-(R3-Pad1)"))
 (segment (start 135 84.848529) (end 122.748529 97.1) (width 0.2) (layer "B.Cu") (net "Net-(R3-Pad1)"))
 (segment (start 135 84.5) (end 135 84.848529) (width 0.2) (layer "B.Cu") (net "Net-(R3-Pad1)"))
 (segment (start 143.5 84) (end 143.8 84) (width 0.2) (layer "F.Cu") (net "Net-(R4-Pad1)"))
 (segment (start 129.497244 97.5) (end 133.5 93.497244) (width 0.2) (layer "F.Cu") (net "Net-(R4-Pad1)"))
 (segment (start 127.175 93) (end 128.1875 94.0125) (width 0.2) (layer "F.Cu") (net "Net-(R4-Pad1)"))
 (segment (start 128.1875 97.184744) (end 128.502756 97.5) (width 0.2) (layer "F.Cu") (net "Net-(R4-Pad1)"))
 (segment (start 128.502756 97.5) (end 129.497244 97.5) (width 0.2) (layer "F.Cu") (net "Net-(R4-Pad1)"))
 (segment (start 143.8 84) (end 145.05 82.75) (width 0.2) (layer "F.Cu") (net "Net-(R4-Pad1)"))
 (segment (start 133.5 93.497244) (end 133.5 92.5) (width 0.2) (layer "F.Cu") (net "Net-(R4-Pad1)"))
 (segment (start 128.1875 94.0125) (end 128.1875 97.184744) (width 0.2) (layer "F.Cu") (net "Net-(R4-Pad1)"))
 (via (at 133.5 92.5) (size 0.6) (drill 0.3) (layers "F.Cu" "B.Cu") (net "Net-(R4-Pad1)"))
 (via (at 143.5 84) (size 0.6) (drill 0.3) (layers "F.Cu" "B.Cu") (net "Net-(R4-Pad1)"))
 (segment (start 133.5 92.5) (end 133.5 89.151471) (width 0.2) (layer "B.Cu") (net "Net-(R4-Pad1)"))
 (segment (start 133.5 89.151471) (end 138.651471 84) (width 0.2) (layer "B.Cu") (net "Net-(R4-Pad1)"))
 (segment (start 138.651471 84) (end 143.5 84) (width 0.2) (layer "B.Cu") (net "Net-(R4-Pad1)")))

